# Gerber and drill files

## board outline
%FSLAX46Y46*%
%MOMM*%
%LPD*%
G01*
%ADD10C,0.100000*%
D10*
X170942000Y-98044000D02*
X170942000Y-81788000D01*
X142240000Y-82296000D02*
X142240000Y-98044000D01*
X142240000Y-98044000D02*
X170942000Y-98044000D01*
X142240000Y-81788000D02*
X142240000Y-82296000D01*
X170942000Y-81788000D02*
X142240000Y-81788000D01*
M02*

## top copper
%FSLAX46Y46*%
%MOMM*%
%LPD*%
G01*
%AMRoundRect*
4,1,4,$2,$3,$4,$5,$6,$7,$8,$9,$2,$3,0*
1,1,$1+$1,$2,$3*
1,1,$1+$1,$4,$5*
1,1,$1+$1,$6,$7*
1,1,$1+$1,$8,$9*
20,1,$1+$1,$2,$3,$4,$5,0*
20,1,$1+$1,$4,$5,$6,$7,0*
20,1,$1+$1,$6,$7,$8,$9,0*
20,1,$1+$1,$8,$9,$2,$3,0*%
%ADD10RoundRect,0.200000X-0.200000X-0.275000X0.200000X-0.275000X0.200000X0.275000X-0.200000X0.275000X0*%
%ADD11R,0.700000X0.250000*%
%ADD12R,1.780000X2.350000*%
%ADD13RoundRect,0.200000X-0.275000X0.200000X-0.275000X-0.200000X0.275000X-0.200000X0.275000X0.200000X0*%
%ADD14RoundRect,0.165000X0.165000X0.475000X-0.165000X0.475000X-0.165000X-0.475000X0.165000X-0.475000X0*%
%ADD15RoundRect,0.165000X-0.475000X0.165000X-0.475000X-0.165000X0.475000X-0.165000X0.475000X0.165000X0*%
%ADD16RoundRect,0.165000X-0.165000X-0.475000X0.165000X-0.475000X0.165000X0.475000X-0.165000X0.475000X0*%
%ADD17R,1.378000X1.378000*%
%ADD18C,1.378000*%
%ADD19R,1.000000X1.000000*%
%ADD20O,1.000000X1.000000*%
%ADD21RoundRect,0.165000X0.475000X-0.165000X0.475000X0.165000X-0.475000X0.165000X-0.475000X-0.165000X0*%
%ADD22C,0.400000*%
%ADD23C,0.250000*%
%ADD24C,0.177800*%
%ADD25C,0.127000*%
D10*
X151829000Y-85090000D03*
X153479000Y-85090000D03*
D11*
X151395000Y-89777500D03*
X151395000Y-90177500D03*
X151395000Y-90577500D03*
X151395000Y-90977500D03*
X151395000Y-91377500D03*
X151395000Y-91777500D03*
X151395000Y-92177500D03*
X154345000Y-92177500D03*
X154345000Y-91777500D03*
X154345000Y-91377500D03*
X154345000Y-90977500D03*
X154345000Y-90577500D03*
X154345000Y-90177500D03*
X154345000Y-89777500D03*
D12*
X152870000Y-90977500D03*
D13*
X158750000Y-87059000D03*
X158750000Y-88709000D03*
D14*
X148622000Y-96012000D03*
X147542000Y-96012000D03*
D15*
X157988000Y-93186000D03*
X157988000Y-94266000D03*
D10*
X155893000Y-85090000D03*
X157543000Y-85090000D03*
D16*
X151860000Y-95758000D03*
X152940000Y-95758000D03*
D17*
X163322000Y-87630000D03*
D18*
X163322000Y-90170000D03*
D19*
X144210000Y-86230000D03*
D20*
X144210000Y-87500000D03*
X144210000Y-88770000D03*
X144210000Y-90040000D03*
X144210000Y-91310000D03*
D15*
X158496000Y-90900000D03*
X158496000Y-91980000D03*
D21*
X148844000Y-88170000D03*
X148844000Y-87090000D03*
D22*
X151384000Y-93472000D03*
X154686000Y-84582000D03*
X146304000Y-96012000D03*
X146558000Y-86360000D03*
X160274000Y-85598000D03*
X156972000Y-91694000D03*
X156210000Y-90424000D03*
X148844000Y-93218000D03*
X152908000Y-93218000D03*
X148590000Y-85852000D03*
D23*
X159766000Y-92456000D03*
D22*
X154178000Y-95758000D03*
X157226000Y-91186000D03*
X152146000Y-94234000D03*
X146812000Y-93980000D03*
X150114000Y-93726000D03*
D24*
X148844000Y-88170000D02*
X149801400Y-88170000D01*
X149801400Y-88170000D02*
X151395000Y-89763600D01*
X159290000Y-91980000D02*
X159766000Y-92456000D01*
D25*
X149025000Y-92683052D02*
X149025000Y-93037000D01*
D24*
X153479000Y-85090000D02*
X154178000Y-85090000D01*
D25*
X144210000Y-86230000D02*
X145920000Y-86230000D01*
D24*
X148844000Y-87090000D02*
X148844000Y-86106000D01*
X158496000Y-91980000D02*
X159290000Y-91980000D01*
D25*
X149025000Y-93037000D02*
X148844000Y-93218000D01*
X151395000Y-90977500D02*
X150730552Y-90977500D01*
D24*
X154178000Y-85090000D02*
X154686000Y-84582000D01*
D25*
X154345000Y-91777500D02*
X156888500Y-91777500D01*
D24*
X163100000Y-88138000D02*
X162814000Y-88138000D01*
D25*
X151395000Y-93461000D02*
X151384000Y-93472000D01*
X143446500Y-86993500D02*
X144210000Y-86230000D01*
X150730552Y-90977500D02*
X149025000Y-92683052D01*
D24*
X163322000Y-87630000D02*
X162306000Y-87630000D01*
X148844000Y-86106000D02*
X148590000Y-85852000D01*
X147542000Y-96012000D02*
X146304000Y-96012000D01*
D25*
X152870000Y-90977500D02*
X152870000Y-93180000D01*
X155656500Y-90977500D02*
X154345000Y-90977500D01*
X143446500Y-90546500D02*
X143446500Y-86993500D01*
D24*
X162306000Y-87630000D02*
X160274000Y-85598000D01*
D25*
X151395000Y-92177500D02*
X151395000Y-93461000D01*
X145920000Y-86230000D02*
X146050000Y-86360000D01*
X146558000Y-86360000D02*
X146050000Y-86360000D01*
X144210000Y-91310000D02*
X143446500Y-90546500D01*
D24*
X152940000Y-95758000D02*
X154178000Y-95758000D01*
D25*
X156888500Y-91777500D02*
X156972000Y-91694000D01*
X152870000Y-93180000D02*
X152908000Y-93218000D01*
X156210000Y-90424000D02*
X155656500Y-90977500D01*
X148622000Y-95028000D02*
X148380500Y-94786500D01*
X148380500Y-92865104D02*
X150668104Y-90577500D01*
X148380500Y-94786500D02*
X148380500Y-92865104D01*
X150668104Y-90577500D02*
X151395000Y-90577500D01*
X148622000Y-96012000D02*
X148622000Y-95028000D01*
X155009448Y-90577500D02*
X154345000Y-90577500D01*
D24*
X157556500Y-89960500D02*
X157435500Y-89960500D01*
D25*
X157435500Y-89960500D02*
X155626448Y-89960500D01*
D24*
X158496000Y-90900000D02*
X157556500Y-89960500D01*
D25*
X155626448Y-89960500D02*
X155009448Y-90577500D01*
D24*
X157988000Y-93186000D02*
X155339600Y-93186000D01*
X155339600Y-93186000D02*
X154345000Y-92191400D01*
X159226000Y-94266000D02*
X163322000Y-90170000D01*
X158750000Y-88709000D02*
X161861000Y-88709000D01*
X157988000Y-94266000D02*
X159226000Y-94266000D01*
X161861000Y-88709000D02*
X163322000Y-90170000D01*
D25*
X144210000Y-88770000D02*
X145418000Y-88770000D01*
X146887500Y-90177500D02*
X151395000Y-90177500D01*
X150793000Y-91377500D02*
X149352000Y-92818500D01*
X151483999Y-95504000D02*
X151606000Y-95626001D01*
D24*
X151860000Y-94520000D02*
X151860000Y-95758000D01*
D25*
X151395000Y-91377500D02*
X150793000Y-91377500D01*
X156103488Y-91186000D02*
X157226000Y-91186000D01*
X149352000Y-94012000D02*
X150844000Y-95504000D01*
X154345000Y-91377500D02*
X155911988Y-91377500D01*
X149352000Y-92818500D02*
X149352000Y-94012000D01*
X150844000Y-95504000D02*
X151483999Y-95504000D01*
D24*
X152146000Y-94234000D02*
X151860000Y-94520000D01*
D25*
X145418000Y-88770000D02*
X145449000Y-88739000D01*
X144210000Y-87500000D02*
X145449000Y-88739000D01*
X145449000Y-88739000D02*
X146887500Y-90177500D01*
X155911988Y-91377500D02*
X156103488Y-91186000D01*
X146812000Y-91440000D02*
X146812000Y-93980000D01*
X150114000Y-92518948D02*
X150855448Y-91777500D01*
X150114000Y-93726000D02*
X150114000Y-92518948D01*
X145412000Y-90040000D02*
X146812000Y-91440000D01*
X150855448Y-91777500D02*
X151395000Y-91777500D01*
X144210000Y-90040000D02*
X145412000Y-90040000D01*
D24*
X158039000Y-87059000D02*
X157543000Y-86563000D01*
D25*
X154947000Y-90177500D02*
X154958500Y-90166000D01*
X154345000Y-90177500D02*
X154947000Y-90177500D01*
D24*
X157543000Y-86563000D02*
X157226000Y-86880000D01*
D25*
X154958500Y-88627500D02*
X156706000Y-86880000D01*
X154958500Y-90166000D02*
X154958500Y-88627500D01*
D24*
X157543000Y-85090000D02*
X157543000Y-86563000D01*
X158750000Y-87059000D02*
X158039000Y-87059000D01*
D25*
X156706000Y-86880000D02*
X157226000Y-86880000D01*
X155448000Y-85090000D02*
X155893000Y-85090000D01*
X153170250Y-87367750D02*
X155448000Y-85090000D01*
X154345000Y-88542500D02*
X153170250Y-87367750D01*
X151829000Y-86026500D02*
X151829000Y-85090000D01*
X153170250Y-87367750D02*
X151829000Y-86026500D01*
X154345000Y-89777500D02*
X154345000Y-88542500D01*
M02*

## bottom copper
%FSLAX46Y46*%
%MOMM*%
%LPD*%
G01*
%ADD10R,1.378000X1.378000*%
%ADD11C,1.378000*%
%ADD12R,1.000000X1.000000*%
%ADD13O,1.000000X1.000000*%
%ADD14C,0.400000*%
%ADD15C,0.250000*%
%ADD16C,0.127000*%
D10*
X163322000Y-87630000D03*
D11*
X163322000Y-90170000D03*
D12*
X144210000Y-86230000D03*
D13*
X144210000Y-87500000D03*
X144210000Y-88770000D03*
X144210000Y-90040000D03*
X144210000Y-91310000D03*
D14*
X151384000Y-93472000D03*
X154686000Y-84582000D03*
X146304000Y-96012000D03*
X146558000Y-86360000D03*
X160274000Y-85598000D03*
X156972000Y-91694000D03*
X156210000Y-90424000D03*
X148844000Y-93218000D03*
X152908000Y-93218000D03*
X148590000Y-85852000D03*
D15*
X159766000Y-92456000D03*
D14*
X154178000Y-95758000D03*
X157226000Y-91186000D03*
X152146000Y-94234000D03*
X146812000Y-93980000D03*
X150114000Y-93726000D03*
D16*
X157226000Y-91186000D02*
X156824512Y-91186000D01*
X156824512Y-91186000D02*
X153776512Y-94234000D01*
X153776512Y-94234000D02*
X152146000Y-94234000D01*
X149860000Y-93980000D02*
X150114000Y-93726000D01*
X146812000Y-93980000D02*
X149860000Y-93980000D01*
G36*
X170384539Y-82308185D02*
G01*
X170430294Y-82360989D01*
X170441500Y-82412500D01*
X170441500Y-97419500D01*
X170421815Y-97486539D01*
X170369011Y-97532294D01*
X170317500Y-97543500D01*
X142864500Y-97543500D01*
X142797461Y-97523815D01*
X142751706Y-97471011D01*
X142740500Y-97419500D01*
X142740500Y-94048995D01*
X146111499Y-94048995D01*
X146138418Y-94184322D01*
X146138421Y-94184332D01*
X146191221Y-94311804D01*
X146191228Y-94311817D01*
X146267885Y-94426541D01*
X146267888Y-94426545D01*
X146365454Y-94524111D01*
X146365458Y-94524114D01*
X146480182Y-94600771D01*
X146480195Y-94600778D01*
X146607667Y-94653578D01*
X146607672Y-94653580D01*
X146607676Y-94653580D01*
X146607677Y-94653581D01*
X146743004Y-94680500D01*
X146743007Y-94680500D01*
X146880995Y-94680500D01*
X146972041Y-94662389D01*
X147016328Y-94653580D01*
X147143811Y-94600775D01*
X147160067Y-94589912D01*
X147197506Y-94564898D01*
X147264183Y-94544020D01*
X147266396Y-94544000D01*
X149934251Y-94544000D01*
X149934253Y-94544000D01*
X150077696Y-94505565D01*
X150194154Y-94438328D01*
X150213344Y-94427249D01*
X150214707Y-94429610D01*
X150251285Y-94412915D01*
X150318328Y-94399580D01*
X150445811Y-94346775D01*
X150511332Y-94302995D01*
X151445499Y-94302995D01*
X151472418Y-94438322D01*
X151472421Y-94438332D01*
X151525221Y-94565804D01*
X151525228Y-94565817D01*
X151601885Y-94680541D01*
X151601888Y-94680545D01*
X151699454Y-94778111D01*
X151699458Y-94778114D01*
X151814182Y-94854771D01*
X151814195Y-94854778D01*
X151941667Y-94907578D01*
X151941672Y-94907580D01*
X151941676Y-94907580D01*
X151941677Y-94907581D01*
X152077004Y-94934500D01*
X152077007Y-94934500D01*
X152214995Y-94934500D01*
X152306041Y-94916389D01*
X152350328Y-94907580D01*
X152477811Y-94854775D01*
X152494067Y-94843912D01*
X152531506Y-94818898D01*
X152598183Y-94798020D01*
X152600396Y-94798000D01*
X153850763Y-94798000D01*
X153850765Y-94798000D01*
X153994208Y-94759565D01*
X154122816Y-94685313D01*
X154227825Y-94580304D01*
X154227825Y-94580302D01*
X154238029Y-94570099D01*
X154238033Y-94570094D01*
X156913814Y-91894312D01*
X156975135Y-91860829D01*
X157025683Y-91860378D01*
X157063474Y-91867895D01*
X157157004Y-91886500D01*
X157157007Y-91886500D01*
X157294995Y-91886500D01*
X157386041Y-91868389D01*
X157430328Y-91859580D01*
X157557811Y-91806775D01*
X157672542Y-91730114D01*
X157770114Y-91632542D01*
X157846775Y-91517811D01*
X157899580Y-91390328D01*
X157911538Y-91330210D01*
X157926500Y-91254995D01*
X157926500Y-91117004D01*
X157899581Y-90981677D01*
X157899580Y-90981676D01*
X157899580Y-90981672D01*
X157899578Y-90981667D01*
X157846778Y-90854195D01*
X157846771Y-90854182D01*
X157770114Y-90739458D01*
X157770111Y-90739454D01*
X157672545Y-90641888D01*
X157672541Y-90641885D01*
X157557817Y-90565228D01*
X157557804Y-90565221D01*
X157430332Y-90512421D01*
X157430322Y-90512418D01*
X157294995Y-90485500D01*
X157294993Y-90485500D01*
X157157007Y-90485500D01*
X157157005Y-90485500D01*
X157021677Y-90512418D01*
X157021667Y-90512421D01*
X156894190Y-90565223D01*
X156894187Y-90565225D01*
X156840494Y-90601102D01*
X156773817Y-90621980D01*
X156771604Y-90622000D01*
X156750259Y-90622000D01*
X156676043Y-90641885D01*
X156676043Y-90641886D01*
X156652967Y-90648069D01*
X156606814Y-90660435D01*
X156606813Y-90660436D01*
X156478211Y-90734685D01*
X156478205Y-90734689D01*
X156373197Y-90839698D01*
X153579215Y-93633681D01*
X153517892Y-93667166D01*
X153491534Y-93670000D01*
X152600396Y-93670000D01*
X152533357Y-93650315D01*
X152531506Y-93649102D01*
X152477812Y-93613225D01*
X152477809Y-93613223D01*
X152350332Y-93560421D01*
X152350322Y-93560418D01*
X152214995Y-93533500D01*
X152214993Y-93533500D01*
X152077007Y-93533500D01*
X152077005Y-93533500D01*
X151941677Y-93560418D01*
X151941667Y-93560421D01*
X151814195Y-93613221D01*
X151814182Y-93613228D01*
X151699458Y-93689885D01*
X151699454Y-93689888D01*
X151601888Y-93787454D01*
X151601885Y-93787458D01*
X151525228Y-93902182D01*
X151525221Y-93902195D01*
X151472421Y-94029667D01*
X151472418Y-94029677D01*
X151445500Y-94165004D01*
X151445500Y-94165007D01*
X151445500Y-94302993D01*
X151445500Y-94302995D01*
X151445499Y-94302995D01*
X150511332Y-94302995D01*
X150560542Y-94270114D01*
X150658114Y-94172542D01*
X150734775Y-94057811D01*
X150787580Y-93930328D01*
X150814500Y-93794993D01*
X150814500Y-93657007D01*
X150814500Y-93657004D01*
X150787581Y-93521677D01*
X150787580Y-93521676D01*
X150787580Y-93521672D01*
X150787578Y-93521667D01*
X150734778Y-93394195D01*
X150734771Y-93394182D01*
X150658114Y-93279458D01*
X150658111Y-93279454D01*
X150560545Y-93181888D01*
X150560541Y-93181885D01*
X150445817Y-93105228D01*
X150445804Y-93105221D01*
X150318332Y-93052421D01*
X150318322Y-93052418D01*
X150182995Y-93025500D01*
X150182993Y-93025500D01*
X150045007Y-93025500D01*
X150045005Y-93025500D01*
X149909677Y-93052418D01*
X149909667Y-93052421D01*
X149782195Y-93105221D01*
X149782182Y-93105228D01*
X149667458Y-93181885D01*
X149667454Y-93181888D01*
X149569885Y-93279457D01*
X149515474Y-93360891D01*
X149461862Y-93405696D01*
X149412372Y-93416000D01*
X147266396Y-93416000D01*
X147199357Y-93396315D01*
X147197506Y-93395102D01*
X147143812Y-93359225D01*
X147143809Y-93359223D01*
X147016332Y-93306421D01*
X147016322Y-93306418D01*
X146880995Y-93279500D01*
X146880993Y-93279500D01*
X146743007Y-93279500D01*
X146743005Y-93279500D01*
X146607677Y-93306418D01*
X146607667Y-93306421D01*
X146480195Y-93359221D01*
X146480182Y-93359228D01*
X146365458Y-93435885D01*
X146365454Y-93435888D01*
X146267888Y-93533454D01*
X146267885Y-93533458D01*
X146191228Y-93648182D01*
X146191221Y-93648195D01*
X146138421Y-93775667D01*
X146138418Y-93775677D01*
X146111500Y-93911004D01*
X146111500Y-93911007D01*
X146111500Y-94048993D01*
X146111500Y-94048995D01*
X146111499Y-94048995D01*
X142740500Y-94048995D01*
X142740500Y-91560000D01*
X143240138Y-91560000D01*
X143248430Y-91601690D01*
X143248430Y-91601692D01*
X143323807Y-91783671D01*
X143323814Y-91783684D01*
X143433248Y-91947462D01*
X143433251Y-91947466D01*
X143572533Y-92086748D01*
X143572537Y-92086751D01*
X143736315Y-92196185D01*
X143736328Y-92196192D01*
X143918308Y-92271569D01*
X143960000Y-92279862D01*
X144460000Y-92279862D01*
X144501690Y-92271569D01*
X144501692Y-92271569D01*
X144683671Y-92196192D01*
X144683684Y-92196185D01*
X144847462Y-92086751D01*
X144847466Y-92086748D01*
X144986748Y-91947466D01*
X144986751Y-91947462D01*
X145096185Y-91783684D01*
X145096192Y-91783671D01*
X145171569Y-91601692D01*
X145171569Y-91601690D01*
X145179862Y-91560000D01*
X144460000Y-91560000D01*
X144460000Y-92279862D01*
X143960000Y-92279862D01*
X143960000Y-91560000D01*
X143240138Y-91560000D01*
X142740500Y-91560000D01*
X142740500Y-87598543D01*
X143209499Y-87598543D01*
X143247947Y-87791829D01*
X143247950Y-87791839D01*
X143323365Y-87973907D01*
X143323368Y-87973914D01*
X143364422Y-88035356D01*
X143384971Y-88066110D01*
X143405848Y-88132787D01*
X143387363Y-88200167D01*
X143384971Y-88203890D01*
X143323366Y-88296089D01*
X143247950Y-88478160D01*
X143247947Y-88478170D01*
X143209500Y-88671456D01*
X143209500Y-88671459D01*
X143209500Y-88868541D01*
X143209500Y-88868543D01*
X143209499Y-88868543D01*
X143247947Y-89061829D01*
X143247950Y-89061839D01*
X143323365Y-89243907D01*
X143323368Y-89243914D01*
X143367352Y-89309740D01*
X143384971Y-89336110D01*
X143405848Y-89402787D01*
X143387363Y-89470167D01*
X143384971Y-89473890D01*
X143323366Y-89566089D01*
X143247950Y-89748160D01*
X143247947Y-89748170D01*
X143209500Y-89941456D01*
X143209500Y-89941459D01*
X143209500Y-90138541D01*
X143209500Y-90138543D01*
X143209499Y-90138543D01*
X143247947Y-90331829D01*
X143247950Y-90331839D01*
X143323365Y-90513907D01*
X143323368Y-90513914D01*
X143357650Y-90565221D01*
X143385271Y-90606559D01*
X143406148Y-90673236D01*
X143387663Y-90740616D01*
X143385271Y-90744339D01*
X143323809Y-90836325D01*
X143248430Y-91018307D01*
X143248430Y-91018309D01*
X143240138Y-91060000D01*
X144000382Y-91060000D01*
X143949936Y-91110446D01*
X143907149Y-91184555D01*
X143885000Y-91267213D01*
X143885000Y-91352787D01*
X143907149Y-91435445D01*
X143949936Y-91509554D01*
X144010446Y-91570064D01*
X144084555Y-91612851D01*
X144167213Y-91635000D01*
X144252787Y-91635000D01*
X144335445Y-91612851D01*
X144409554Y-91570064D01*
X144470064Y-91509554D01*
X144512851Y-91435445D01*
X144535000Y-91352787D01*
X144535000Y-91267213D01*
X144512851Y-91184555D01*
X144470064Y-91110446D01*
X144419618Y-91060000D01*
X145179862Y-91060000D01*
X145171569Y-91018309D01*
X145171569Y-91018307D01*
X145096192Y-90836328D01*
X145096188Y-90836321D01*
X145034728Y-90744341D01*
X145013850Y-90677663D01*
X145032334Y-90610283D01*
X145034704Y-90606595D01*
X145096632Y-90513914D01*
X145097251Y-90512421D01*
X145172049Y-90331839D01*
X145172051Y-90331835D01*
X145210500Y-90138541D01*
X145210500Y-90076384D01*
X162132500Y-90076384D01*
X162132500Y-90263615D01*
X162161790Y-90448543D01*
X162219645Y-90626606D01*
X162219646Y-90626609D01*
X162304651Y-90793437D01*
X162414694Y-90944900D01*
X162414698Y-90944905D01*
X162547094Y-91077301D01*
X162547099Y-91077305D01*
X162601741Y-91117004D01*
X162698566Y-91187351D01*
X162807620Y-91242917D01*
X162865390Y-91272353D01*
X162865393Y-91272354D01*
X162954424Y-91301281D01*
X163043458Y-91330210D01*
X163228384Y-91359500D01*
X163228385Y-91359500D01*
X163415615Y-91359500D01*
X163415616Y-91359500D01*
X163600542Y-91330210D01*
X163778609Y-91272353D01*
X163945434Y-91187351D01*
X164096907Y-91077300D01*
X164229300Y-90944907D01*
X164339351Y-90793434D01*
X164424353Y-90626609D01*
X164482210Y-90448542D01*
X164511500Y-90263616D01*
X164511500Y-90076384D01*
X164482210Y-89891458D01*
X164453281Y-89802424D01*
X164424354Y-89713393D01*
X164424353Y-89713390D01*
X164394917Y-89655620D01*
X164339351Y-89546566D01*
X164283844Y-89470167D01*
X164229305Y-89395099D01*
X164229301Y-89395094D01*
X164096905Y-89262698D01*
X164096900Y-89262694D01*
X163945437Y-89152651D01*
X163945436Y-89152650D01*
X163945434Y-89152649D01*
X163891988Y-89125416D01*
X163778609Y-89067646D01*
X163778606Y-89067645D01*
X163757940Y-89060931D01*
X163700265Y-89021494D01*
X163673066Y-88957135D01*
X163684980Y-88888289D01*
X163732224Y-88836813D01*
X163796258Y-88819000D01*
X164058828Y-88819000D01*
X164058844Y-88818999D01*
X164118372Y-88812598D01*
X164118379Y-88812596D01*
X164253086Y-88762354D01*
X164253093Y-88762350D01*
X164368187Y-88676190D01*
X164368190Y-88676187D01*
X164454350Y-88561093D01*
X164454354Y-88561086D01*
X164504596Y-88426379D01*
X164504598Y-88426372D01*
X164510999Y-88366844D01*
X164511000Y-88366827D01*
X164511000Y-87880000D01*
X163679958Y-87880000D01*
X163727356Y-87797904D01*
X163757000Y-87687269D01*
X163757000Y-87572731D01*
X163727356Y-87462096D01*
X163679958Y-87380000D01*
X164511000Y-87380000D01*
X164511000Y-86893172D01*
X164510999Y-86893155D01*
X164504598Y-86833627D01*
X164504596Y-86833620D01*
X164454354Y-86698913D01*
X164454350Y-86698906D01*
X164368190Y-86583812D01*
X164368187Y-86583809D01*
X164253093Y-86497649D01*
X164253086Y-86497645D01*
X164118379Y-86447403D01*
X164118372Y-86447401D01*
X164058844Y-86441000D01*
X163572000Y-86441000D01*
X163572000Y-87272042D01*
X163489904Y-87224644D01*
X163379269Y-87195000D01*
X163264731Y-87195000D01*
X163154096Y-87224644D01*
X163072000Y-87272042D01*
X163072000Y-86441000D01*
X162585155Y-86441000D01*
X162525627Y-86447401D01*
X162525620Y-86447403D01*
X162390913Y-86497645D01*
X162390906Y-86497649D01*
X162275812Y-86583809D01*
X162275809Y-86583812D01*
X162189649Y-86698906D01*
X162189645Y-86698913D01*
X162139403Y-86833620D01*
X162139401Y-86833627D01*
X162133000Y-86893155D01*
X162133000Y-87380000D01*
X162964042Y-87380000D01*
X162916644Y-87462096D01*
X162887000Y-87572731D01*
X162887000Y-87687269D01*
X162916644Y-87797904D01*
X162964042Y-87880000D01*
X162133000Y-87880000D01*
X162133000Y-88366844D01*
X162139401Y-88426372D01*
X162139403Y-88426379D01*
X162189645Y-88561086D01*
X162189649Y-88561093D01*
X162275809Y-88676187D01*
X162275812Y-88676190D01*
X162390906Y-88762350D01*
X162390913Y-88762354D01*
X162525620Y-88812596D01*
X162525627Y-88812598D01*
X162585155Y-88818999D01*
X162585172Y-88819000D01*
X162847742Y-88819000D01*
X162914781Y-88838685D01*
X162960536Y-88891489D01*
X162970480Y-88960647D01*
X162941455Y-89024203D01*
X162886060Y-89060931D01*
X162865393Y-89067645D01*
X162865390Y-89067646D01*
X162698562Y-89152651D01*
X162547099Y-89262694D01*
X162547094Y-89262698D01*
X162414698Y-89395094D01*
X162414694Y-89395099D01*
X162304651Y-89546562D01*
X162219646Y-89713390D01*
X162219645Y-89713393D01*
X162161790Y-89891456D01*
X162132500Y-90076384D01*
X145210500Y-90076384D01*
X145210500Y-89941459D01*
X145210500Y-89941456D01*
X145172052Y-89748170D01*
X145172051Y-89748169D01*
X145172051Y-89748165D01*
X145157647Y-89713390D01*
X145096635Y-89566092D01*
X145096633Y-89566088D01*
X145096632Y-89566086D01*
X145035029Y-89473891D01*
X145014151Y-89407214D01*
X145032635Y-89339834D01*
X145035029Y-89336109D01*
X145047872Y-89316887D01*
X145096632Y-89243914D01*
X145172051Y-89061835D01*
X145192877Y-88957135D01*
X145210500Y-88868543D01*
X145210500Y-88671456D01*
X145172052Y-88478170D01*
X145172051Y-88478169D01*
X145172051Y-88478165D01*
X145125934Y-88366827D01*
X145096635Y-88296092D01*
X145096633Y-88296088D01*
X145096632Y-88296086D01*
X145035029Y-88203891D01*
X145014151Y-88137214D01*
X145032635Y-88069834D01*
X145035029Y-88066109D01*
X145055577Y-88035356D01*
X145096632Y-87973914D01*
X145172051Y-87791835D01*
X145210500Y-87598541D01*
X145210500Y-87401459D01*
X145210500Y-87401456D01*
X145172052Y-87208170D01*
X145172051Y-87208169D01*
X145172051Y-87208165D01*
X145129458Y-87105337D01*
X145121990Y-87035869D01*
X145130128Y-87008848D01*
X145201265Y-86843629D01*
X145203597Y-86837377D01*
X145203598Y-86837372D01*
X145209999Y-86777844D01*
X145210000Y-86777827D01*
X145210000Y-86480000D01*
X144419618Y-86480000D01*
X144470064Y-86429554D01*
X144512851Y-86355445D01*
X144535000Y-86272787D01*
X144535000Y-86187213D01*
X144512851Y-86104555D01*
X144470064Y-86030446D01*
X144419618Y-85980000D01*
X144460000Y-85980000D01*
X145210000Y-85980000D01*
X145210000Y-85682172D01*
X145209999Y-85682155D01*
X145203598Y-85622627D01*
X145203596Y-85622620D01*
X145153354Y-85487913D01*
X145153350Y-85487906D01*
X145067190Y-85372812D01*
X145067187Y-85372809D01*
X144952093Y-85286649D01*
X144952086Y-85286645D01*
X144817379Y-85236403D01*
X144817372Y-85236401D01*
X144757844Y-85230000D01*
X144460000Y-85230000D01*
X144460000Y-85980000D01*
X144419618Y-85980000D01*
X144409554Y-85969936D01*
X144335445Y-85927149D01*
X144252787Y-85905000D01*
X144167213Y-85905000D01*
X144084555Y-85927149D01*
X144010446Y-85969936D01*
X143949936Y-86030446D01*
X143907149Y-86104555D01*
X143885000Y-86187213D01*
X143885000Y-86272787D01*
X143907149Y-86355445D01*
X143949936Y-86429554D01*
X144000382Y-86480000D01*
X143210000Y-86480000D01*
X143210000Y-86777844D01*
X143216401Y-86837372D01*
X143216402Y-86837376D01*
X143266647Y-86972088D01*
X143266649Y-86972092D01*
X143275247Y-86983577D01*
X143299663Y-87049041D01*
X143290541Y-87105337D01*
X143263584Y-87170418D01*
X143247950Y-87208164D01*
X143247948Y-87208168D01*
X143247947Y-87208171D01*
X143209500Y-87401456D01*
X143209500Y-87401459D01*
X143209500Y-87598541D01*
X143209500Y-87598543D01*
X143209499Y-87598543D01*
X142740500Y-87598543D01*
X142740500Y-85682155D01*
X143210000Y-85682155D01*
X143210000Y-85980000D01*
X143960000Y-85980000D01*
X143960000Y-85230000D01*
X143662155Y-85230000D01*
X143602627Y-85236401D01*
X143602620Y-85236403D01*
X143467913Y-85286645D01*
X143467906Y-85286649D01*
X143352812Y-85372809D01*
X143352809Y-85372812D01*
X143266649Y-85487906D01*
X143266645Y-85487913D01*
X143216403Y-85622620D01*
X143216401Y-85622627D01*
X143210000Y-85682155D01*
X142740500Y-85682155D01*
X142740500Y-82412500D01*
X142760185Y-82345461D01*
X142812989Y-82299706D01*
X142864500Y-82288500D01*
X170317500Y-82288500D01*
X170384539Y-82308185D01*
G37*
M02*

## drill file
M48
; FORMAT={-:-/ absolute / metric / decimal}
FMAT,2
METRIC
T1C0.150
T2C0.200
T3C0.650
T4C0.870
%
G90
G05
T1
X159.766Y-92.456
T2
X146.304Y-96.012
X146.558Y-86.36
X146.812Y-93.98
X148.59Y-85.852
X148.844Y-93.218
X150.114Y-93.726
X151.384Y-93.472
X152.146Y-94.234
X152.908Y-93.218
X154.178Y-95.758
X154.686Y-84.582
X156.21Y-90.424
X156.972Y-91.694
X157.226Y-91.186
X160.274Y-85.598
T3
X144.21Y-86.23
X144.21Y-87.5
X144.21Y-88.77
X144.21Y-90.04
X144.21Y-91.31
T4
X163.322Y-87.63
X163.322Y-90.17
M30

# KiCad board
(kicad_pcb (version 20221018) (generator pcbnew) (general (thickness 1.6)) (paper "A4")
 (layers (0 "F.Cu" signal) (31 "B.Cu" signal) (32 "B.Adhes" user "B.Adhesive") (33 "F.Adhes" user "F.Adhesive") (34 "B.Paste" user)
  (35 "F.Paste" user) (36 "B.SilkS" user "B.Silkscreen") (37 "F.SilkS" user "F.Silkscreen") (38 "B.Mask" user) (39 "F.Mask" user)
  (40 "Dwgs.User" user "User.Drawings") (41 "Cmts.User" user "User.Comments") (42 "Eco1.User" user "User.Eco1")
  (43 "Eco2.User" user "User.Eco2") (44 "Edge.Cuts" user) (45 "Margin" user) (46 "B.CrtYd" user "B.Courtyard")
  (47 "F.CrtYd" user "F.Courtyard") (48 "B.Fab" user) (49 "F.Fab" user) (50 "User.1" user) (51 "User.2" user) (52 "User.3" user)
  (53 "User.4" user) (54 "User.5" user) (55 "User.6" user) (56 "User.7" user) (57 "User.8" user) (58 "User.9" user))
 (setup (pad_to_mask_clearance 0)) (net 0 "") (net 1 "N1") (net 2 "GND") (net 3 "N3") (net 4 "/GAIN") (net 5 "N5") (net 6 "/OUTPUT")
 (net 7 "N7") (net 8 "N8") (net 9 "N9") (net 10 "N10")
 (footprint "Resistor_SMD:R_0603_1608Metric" (layer "F.Cu") (at 152.654 85.09)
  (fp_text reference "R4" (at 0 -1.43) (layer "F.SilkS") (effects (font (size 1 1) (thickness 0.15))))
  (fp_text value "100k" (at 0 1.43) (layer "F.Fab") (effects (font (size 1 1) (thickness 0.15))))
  (pad "1" smd roundrect (at -0.825 0) (size 0.8 0.95) (layers "F.Cu" "F.Paste" "F.Mask") (roundrect_rratio 0.25) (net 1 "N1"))
  (pad "2" smd roundrect (at 0.825 0) (size 0.8 0.95) (layers "F.Cu" "F.Paste" "F.Mask") (roundrect_rratio 0.25) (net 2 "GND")))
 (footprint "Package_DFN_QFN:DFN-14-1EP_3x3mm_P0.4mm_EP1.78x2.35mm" (layer "F.Cu") (at 152.87 90.9775)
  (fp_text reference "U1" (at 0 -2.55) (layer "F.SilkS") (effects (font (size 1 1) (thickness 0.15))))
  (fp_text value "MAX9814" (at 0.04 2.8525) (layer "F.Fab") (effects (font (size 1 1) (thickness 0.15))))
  (pad "" smd rect (at -0.445 -0.5875) (size 0.7 0.97) (layers "F.Paste"))
  (pad "" smd rect (at -0.445 0.5875) (size 0.7 0.97) (layers "F.Paste"))
  (pad "" smd rect (at 0.45 -0.5875) (size 0.7 0.97) (layers "F.Paste"))
  (pad "" smd rect (at 0.45 0.5875) (size 0.7 0.97) (layers "F.Paste"))
  (pad "1" smd rect (at -1.475 -1.2) (size 0.7 0.25) (layers "F.Cu" "F.Paste" "F.Mask") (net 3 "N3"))
  (pad "2" smd rect (at -1.475 -0.8) (size 0.7 0.25) (layers "F.Cu" "F.Paste" "F.Mask") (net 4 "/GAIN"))
  (pad "3" smd rect (at -1.475 -0.4) (size 0.7 0.25) (layers "F.Cu" "F.Paste" "F.Mask") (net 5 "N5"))
  (pad "4" smd rect (at -1.475 0) (size 0.7 0.25) (layers "F.Cu" "F.Paste" "F.Mask") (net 2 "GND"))
  (pad "5" smd rect (at -1.475 0.4) (size 0.7 0.25) (layers "F.Cu" "F.Paste" "F.Mask") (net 4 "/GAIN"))
  (pad "6" smd rect (at -1.475 0.8) (size 0.7 0.25) (layers "F.Cu" "F.Paste" "F.Mask") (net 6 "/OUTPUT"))
  (pad "7" smd rect (at -1.475 1.2) (size 0.7 0.25) (layers "F.Cu" "F.Paste" "F.Mask") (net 2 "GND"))
  (pad "8" smd rect (at 1.475 1.2) (size 0.7 0.25) (layers "F.Cu" "F.Paste" "F.Mask") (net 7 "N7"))
  (pad "9" smd rect (at 1.475 0.8) (size 0.7 0.25) (layers "F.Cu" "F.Paste" "F.Mask") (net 2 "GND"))
  (pad "10" smd rect (at 1.475 0.4) (size 0.7 0.25) (layers "F.Cu" "F.Paste" "F.Mask") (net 4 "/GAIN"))
  (pad "11" smd rect (at 1.475 0) (size 0.7 0.25) (layers "F.Cu" "F.Paste" "F.Mask") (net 2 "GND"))
  (pad "12" smd rect (at 1.475 -0.4) (size 0.7 0.25) (layers "F.Cu" "F.Paste" "F.Mask") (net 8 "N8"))
  (pad "13" smd rect (at 1.475 -0.8) (size 0.7 0.25) (layers "F.Cu" "F.Paste" "F.Mask") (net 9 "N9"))
  (pad "14" smd rect (at 1.475 -1.2) (size 0.7 0.25) (layers "F.Cu" "F.Paste" "F.Mask") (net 1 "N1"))
  (pad "15" smd rect (at 0 0) (size 1.78 2.35) (layers "F.Cu" "F.Mask") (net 2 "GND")))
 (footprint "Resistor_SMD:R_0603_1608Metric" (layer "F.Cu") (at 158.75 87.884 -90)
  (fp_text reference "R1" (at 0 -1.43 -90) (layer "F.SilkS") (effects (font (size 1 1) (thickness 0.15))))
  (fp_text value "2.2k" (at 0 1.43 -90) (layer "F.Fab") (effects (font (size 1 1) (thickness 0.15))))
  (pad "1" smd roundrect (at -0.825 0 270) (size 0.8 0.95) (layers "F.Cu" "F.Paste" "F.Mask") (roundrect_rratio 0.25) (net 9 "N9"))
  (pad "2" smd roundrect (at 0.825 0 270) (size 0.8 0.95) (layers "F.Cu" "F.Paste" "F.Mask") (roundrect_rratio 0.25) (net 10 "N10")))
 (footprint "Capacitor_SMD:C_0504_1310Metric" (layer "F.Cu") (at 148.082 96.012 180)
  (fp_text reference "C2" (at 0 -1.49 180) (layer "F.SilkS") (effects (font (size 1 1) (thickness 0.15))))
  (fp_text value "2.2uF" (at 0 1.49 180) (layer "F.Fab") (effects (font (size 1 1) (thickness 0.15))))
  (pad "1" smd roundrect (at -0.54 0 180) (size 0.66 1.28) (layers "F.Cu" "F.Paste" "F.Mask") (roundrect_rratio 0.25) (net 5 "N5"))
  (pad "2" smd roundrect (at 0.54 0 180) (size 0.66 1.28) (layers "F.Cu" "F.Paste" "F.Mask") (roundrect_rratio 0.25) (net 2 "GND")))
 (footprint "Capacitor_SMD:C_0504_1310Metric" (layer "F.Cu") (at 157.988 93.726 -90)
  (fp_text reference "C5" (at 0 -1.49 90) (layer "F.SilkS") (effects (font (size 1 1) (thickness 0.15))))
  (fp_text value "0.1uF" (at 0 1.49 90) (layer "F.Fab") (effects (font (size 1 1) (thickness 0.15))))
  (pad "1" smd roundrect (at -0.54 0 270) (size 0.66 1.28) (layers "F.Cu" "F.Paste" "F.Mask") (roundrect_rratio 0.25) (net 7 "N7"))
  (pad "2" smd roundrect (at 0.54 0 270) (size 0.66 1.28) (layers "F.Cu" "F.Paste" "F.Mask") (roundrect_rratio 0.25) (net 10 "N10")))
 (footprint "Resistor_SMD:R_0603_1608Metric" (layer "F.Cu") (at 156.718 85.09)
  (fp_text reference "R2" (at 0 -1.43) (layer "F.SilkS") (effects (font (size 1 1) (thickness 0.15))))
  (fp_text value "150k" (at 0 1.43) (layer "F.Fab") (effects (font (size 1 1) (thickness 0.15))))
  (pad "1" smd roundrect (at -0.825 0) (size 0.8 0.95) (layers "F.Cu" "F.Paste" "F.Mask") (roundrect_rratio 0.25) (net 1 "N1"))
  (pad "2" smd roundrect (at 0.825 0) (size 0.8 0.95) (layers "F.Cu" "F.Paste" "F.Mask") (roundrect_rratio 0.25) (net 9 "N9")))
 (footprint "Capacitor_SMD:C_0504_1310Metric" (layer "F.Cu") (at 152.4 95.758)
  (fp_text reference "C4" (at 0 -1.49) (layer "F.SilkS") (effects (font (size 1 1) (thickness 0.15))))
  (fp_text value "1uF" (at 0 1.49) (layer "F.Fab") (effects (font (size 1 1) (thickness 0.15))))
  (pad "1" smd roundrect (at -0.54 0) (size 0.66 1.28) (layers "F.Cu" "F.Paste" "F.Mask") (roundrect_rratio 0.25) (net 4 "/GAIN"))
  (pad "2" smd roundrect (at 0.54 0) (size 0.66 1.28) (layers "F.Cu" "F.Paste" "F.Mask") (roundrect_rratio 0.25) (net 2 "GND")))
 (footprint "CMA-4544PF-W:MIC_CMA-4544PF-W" (layer "F.Cu") (at 165.322 88.9 180)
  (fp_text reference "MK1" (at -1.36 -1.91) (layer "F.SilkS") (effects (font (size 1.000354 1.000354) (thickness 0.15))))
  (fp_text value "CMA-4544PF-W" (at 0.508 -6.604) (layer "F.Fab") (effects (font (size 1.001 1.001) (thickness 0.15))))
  (pad "1" thru_hole rect (at 2 1.27 180) (size 1.378 1.378) (drill 0.87) (layers "*.Cu" "*.Mask") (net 2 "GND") (solder_mask_margin 0.102))
  (pad "2" thru_hole circle (at 2 -1.27 180) (size 1.378 1.378) (drill 0.87) (layers "*.Cu" "*.Mask") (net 10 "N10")
   (solder_mask_margin 0.102)))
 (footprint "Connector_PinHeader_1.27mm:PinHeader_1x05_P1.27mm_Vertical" (layer "F.Cu") (at 144.21 86.23)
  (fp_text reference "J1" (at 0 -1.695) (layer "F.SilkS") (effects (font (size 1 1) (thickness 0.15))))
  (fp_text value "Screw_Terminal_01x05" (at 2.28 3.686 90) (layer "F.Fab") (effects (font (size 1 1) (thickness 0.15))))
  (pad "1" thru_hole rect (at 0 0) (size 1 1) (drill 0.65) (layers "*.Cu" "*.Mask") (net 2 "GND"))
  (pad "2" thru_hole oval (at 0 1.27) (size 1 1) (drill 0.65) (layers "*.Cu" "*.Mask") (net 4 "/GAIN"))
  (pad "3" thru_hole oval (at 0 2.54) (size 1 1) (drill 0.65) (layers "*.Cu" "*.Mask") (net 4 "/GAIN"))
  (pad "4" thru_hole oval (at 0 3.81) (size 1 1) (drill 0.65) (layers "*.Cu" "*.Mask") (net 6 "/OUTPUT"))
  (pad "5" thru_hole oval (at 0 5.08) (size 1 1) (drill 0.65) (layers "*.Cu" "*.Mask") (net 2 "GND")))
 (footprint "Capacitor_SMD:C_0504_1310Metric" (layer "F.Cu") (at 158.496 91.44 -90)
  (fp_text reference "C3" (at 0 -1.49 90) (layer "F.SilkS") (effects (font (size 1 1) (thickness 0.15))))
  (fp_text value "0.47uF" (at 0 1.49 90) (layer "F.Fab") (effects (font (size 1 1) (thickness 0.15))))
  (pad "1" smd roundrect (at -0.54 0 270) (size 0.66 1.28) (layers "F.Cu" "F.Paste" "F.Mask") (roundrect_rratio 0.25) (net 8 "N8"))
  (pad "2" smd roundrect (at 0.54 0 270) (size 0.66 1.28) (layers "F.Cu" "F.Paste" "F.Mask") (roundrect_rratio 0.25) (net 2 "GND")))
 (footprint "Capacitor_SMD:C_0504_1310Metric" (layer "F.Cu") (at 148.844 87.63 90)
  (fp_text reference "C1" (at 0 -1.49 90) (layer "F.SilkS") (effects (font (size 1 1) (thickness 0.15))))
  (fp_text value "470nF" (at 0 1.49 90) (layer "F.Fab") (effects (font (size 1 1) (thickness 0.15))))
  (pad "1" smd roundrect (at -0.54 0 90) (size 0.66 1.28) (layers "F.Cu" "F.Paste" "F.Mask") (roundrect_rratio 0.25) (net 3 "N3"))
  (pad "2" smd roundrect (at 0.54 0 90) (size 0.66 1.28) (layers "F.Cu" "F.Paste" "F.Mask") (roundrect_rratio 0.25) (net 2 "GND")))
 (gr_line (start 170.942 98.044) (end 170.942 81.788) (stroke (width 0.1) (type default)) (layer "Edge.Cuts"))
 (gr_line (start 142.24 82.296) (end 142.24 98.044) (stroke (width 0.1) (type default)) (layer "Edge.Cuts"))
 (gr_line (start 142.24 98.044) (end 170.942 98.044) (stroke (width 0.1) (type default)) (layer "Edge.Cuts"))
 (gr_line (start 142.24 81.788) (end 142.24 82.296) (stroke (width 0.1) (type default)) (layer "Edge.Cuts"))
 (gr_line (start 170.942 81.788) (end 142.24 81.788) (stroke (width 0.1) (type default)) (layer "Edge.Cuts"))
 (segment (start 148.844 88.17) (end 149.8014 88.17) (width 0.1778) (layer "F.Cu") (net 3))
 (segment (start 149.8014 88.17) (end 151.395 89.7636) (width 0.1778) (layer "F.Cu") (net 3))
 (segment (start 159.29 91.98) (end 159.766 92.456) (width 0.1778) (layer "F.Cu") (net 2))
 (segment (start 149.025 92.683052) (end 149.025 93.037) (width 0.127) (layer "F.Cu") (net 2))
 (segment (start 153.479 85.09) (end 154.178 85.09) (width 0.1778) (layer "F.Cu") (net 2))
 (segment (start 144.21 86.23) (end 145.92 86.23) (width 0.127) (layer "F.Cu") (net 2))
 (segment (start 148.844 87.09) (end 148.844 86.106) (width 0.1778) (layer "F.Cu") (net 2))
 (segment (start 158.496 91.98) (end 159.29 91.98) (width 0.1778) (layer "F.Cu") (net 2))
 (segment (start 149.025 93.037) (end 148.844 93.218) (width 0.127) (layer "F.Cu") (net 2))
 (segment (start 151.395 90.9775) (end 150.730552 90.9775) (width 0.127) (layer "F.Cu") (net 2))
 (segment (start 154.178 85.09) (end 154.686 84.582) (width 0.1778) (layer "F.Cu") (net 2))
 (segment (start 154.345 91.7775) (end 156.8885 91.7775) (width 0.127) (layer "F.Cu") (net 2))
 (segment (start 163.1 88.138) (end 162.814 88.138) (width 0.1778) (layer "F.Cu") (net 2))
 (segment (start 151.395 93.461) (end 151.384 93.472) (width 0.127) (layer "F.Cu") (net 2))
 (segment (start 143.4465 86.9935) (end 144.21 86.23) (width 0.127) (layer "F.Cu") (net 2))
 (segment (start 150.730552 90.9775) (end 149.025 92.683052) (width 0.127) (layer "F.Cu") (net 2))
 (segment (start 163.322 87.63) (end 162.306 87.63) (width 0.1778) (layer "F.Cu") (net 2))
 (segment (start 148.844 86.106) (end 148.59 85.852) (width 0.1778) (layer "F.Cu") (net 2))
 (segment (start 147.542 96.012) (end 146.304 96.012) (width 0.1778) (layer "F.Cu") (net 2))
 (segment (start 152.87 90.9775) (end 152.87 93.18) (width 0.127) (layer "F.Cu") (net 2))
 (segment (start 155.6565 90.9775) (end 154.345 90.9775) (width 0.127) (layer "F.Cu") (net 2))
 (segment (start 143.4465 90.5465) (end 143.4465 86.9935) (width 0.127) (layer "F.Cu") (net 2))
 (segment (start 162.306 87.63) (end 160.274 85.598) (width 0.1778) (layer "F.Cu") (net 2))
 (segment (start 151.395 92.1775) (end 151.395 93.461) (width 0.127) (layer "F.Cu") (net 2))
 (segment (start 145.92 86.23) (end 146.05 86.36) (width 0.127) (layer "F.Cu") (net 2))
 (segment (start 146.558 86.36) (end 146.05 86.36) (width 0.127) (layer "F.Cu") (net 2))
 (segment (start 144.21 91.31) (end 143.4465 90.5465) (width 0.127) (layer "F.Cu") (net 2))
 (segment (start 152.94 95.758) (end 154.178 95.758) (width 0.1778) (layer "F.Cu") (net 2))
 (segment (start 156.8885 91.7775) (end 156.972 91.694) (width 0.127) (layer "F.Cu") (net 2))
 (segment (start 152.87 93.18) (end 152.908 93.218) (width 0.127) (layer "F.Cu") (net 2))
 (segment (start 156.21 90.424) (end 155.6565 90.9775) (width 0.127) (layer "F.Cu") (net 2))
 (via (at 151.384 93.472) (size 0.4) (drill 0.2) (layers "F.Cu" "B.Cu") (free) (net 2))
 (via (at 154.686 84.582) (size 0.4) (drill 0.2) (layers "F.Cu" "B.Cu") (free) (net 2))
 (via (at 146.304 96.012) (size 0.4) (drill 0.2) (layers "F.Cu" "B.Cu") (free) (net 2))
 (via (at 146.558 86.36) (size 0.4) (drill 0.2) (layers "F.Cu" "B.Cu") (free) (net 2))
 (via (at 160.274 85.598) (size 0.4) (drill 0.2) (layers "F.Cu" "B.Cu") (free) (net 2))
 (via (at 156.972 91.694) (size 0.4) (drill 0.2) (layers "F.Cu" "B.Cu") (free) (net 2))
 (via (at 156.21 90.424) (size 0.4) (drill 0.2) (layers "F.Cu" "B.Cu") (free) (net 2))
 (via (at 148.844 93.218) (size 0.4) (drill 0.2) (layers "F.Cu" "B.Cu") (free) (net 2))
 (via (at 152.908 93.218) (size 0.4) (drill 0.2) (layers "F.Cu" "B.Cu") (free) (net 2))
 (via (at 148.59 85.852) (size 0.4) (drill 0.2) (layers "F.Cu" "B.Cu") (free) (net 2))
 (via (at 159.766 92.456) (size 0.25) (drill 0.15) (layers "F.Cu" "B.Cu") (free) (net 2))
 (via (at 154.178 95.758) (size 0.4) (drill 0.2) (layers "F.Cu" "B.Cu") (free) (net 2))
 (segment (start 148.622 95.028) (end 148.3805 94.7865) (width 0.127) (layer "F.Cu") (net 5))
 (segment (start 148.3805 92.865104) (end 150.668104 90.5775) (width 0.127) (layer "F.Cu") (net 5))
 (segment (start 148.3805 94.7865) (end 148.3805 92.865104) (width 0.127) (layer "F.Cu") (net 5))
 (segment (start 150.668104 90.5775) (end 151.395 90.5775) (width 0.127) (layer "F.Cu") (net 5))
 (segment (start 148.622 96.012) (end 148.622 95.028) (width 0.127) (layer "F.Cu") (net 5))
 (segment (start 155.009448 90.5775) (end 154.345 90.5775) (width 0.127) (layer "F.Cu") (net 8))
 (segment (start 157.5565 89.9605) (end 157.4355 89.9605) (width 0.1778) (layer "F.Cu") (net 8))
 (segment (start 157.4355 89.9605) (end 155.626448 89.9605) (width 0.127) (layer "F.Cu") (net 8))
 (segment (start 158.496 90.9) (end 157.5565 89.9605) (width 0.1778) (layer "F.Cu") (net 8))
 (segment (start 155.626448 89.9605) (end 155.009448 90.5775) (width 0.127) (layer "F.Cu") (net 8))
 (segment (start 157.988 93.186) (end 155.3396 93.186) (width 0.1778) (layer "F.Cu") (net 7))
 (segment (start 155.3396 93.186) (end 154.345 92.1914) (width 0.1778) (layer "F.Cu") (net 7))
 (segment (start 159.226 94.266) (end 163.322 90.17) (width 0.1778) (layer "F.Cu") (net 10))
 (segment (start 158.75 88.709) (end 161.861 88.709) (width 0.1778) (layer "F.Cu") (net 10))
 (segment (start 157.988 94.266) (end 159.226 94.266) (width 0.1778) (layer "F.Cu") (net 10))
 (segment (start 161.861 88.709) (end 163.322 90.17) (width 0.1778) (layer "F.Cu") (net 10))
 (segment (start 144.21 88.77) (end 145.418 88.77) (width 0.127) (layer "F.Cu") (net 4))
 (segment (start 146.8875 90.1775) (end 151.395 90.1775) (width 0.127) (layer "F.Cu") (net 4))
 (segment (start 150.793 91.3775) (end 149.352 92.8185) (width 0.127) (layer "F.Cu") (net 4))
 (segment (start 151.483999 95.504) (end 151.606 95.626001) (width 0.127) (layer "F.Cu") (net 4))
 (segment (start 151.86 94.52) (end 151.86 95.758) (width 0.1778) (layer "F.Cu") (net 4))
 (segment (start 151.395 91.3775) (end 150.793 91.3775) (width 0.127) (layer "F.Cu") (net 4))
 (segment (start 156.103488 91.186) (end 157.226 91.186) (width 0.127) (layer "F.Cu") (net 4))
 (segment (start 149.352 94.012) (end 150.844 95.504) (width 0.127) (layer "F.Cu") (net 4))
 (segment (start 154.345 91.3775) (end 155.911988 91.3775) (width 0.127) (layer "F.Cu") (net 4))
 (segment (start 149.352 92.8185) (end 149.352 94.012) (width 0.127) (layer "F.Cu") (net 4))
 (segment (start 150.844 95.504) (end 151.483999 95.504) (width 0.127) (layer "F.Cu") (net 4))
 (segment (start 152.146 94.234) (end 151.86 94.52) (width 0.1778) (layer "F.Cu") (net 4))
 (segment (start 145.418 88.77) (end 145.449 88.739) (width 0.127) (layer "F.Cu") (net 4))
 (segment (start 144.21 87.5) (end 145.449 88.739) (width 0.127) (layer "F.Cu") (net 4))
 (segment (start 145.449 88.739) (end 146.8875 90.1775) (width 0.127) (layer "F.Cu") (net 4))
 (segment (start 155.911988 91.3775) (end 156.103488 91.186) (width 0.127) (layer "F.Cu") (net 4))
 (via (at 157.226 91.186) (size 0.4) (drill 0.2) (layers "F.Cu" "B.Cu") (free) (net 4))
 (via (at 152.146 94.234) (size 0.4) (drill 0.2) (layers "F.Cu" "B.Cu") (free) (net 4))
 (segment (start 157.226 91.186) (end 156.824512 91.186) (width 0.127) (layer "B.Cu") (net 4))
 (segment (start 156.824512 91.186) (end 153.776512 94.234) (width 0.127) (layer "B.Cu") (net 4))
 (segment (start 153.776512 94.234) (end 152.146 94.234) (width 0.127) (layer "B.Cu") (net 4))
 (segment (start 146.812 91.44) (end 146.812 93.98) (width 0.127) (layer "F.Cu") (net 6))
 (segment (start 150.114 92.518948) (end 150.855448 91.7775) (width 0.127) (layer "F.Cu") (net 6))
 (segment (start 150.114 93.726) (end 150.114 92.518948) (width 0.127) (layer "F.Cu") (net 6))
 (segment (start 145.412 90.04) (end 146.812 91.44) (width 0.127) (layer "F.Cu") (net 6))
 (segment (start 150.855448 91.7775) (end 151.395 91.7775) (width 0.127) (layer "F.Cu") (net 6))
 (segment (start 144.21 90.04) (end 145.412 90.04) (width 0.127) (layer "F.Cu") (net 6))
 (via (at 146.812 93.98) (size 0.4) (drill 0.2) (layers "F.Cu" "B.Cu") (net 6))
 (via (at 150.114 93.726) (size 0.4) (drill 0.2) (layers "F.Cu" "B.Cu") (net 6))
 (segment (start 149.86 93.98) (end 150.114 93.726) (width 0.127) (layer "B.Cu") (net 6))
 (segment (start 146.812 93.98) (end 149.86 93.98) (width 0.127) (layer "B.Cu") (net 6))
 (segment (start 158.039 87.059) (end 157.543 86.563) (width 0.1778) (layer "F.Cu") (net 9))
 (segment (start 154.947 90.1775) (end 154.9585 90.166) (width 0.127) (layer "F.Cu") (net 9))
 (segment (start 154.345 90.1775) (end 154.947 90.1775) (width 0.127) (layer "F.Cu") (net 9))
 (segment (start 157.543 86.563) (end 157.226 86.88) (width 0.1778) (layer "F.Cu") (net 9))
 (segment (start 154.9585 88.6275) (end 156.706 86.88) (width 0.127) (layer "F.Cu") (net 9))
 (segment (start 154.9585 90.166) (end 154.9585 88.6275) (width 0.127) (layer "F.Cu") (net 9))
 (segment (start 157.543 85.09) (end 157.543 86.563) (width 0.1778) (layer "F.Cu") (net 9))
 (segment (start 158.75 87.059) (end 158.039 87.059) (width 0.1778) (layer "F.Cu") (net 9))
 (segment (start 156.706 86.88) (end 157.226 86.88) (width 0.127) (layer "F.Cu") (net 9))
 (segment (start 155.448 85.09) (end 155.893 85.09) (width 0.127) (layer "F.Cu") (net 1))
 (segment (start 153.17025 87.36775) (end 155.448 85.09) (width 0.127) (layer "F.Cu") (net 1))
 (segment (start 154.345 88.5425) (end 153.17025 87.36775) (width 0.127) (layer "F.Cu") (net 1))
 (segment (start 151.829 86.0265) (end 151.829 85.09) (width 0.127) (layer "F.Cu") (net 1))
 (segment (start 153.17025 87.36775) (end 151.829 86.0265) (width 0.127) (layer "F.Cu") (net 1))
 (segment (start 154.345 89.7775) (end 154.345 88.5425) (width 0.127) (layer "F.Cu") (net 1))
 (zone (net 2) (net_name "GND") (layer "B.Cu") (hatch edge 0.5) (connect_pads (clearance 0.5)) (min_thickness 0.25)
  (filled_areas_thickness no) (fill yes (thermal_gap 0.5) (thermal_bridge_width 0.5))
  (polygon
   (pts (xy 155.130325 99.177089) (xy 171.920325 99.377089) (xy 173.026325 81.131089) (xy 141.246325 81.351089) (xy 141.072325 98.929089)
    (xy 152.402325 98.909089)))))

